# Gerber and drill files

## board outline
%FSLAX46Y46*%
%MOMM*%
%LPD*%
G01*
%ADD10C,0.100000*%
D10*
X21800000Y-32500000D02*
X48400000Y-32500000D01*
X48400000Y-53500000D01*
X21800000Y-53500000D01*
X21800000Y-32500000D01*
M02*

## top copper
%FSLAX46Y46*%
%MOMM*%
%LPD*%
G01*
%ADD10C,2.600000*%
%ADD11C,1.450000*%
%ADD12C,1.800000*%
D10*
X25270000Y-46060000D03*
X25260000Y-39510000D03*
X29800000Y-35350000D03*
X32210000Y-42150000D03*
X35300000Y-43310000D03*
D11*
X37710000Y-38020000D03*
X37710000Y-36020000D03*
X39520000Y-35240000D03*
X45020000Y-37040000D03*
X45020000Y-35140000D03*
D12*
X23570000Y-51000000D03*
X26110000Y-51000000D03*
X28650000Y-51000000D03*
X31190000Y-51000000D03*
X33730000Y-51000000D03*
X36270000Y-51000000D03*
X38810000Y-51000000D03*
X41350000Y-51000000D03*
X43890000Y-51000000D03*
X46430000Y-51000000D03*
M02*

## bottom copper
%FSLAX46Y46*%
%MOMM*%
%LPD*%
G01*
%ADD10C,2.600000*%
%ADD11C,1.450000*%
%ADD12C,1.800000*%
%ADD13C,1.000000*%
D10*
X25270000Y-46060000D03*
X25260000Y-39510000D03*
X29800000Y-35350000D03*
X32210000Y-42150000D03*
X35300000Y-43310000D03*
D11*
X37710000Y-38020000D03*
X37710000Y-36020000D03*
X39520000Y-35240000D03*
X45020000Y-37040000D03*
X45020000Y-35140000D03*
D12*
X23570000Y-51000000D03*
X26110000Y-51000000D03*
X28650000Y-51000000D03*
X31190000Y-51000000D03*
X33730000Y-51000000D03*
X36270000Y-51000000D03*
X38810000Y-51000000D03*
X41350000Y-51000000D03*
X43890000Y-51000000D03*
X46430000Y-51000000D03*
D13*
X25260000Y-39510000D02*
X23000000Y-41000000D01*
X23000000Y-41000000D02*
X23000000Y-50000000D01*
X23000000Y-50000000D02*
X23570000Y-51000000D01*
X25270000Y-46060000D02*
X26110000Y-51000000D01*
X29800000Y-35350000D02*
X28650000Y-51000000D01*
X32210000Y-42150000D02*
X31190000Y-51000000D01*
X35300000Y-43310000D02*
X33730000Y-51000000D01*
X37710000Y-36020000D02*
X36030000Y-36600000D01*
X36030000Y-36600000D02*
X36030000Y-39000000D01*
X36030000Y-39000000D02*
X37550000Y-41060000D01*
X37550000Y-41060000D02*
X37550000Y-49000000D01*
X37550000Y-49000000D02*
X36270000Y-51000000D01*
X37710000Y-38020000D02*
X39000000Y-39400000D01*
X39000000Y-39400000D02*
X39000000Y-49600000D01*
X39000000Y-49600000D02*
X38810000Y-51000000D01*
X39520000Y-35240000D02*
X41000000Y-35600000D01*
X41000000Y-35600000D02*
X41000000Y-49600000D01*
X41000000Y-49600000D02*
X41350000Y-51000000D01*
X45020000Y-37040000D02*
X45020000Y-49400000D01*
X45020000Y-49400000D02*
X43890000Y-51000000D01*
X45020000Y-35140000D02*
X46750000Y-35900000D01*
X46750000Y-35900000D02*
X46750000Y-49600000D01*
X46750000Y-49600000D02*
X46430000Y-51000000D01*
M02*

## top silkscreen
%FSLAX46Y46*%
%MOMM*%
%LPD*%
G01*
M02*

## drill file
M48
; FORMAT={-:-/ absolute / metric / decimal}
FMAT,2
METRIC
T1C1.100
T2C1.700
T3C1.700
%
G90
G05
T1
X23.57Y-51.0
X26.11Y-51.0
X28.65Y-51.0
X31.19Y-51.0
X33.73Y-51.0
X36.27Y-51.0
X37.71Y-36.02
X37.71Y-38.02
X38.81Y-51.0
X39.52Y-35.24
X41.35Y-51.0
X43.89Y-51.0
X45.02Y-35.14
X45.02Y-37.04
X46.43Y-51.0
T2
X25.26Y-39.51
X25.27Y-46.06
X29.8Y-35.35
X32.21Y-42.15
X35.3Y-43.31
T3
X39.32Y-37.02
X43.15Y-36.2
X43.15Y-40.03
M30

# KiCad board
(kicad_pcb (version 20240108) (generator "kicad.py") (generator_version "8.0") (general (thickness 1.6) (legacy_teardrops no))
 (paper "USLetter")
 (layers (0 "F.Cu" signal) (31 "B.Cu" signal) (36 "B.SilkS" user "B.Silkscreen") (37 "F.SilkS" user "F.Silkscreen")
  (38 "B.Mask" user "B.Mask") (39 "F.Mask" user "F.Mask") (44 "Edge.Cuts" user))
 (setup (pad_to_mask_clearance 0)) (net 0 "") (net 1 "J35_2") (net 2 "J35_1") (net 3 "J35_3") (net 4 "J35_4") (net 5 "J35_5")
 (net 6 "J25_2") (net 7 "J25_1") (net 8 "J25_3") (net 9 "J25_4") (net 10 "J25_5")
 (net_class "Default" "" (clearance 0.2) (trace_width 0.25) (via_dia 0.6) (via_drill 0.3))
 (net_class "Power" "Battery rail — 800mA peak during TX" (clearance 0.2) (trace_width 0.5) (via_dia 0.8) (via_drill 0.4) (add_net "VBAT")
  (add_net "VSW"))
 (segment (start 25.26 39.51) (end 23.0 41.0) (width 1.0) (layer "B.Cu") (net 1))
 (segment (start 23.0 41.0) (end 23.0 50.0) (width 1.0) (layer "B.Cu") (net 1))
 (segment (start 23.0 50.0) (end 23.57 51.0) (width 1.0) (layer "B.Cu") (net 1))
 (segment (start 25.27 46.06) (end 26.11 51.0) (width 1.0) (layer "B.Cu") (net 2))
 (segment (start 29.8 35.35) (end 28.65 51.0) (width 1.0) (layer "B.Cu") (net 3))
 (segment (start 32.21 42.15) (end 31.19 51.0) (width 1.0) (layer "B.Cu") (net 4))
 (segment (start 35.3 43.31) (end 33.73 51.0) (width 1.0) (layer "B.Cu") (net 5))
 (segment (start 37.71 36.02) (end 36.03 36.6) (width 1.0) (layer "B.Cu") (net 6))
 (segment (start 36.03 36.6) (end 36.03 39.0) (width 1.0) (layer "B.Cu") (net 6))
 (segment (start 36.03 39.0) (end 37.55 41.06) (width 1.0) (layer "B.Cu") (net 6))
 (segment (start 37.55 41.06) (end 37.55 49.0) (width 1.0) (layer "B.Cu") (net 6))
 (segment (start 37.55 49.0) (end 36.27 51.0) (width 1.0) (layer "B.Cu") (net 6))
 (segment (start 37.71 38.02) (end 39.0 39.4) (width 1.0) (layer "B.Cu") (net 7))
 (segment (start 39.0 39.4) (end 39.0 49.6) (width 1.0) (layer "B.Cu") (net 7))
 (segment (start 39.0 49.6) (end 38.81 51.0) (width 1.0) (layer "B.Cu") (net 7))
 (segment (start 39.52 35.24) (end 41.0 35.6) (width 1.0) (layer "B.Cu") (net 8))
 (segment (start 41.0 35.6) (end 41.0 49.6) (width 1.0) (layer "B.Cu") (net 8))
 (segment (start 41.0 49.6) (end 41.35 51.0) (width 1.0) (layer "B.Cu") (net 8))
 (segment (start 45.02 37.04) (end 45.02 49.4) (width 1.0) (layer "B.Cu") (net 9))
 (segment (start 45.02 49.4) (end 43.89 51.0) (width 1.0) (layer "B.Cu") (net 9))
 (segment (start 45.02 35.14) (end 46.75 35.9) (width 1.0) (layer "B.Cu") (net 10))
 (segment (start 46.75 35.9) (end 46.75 49.6) (width 1.0) (layer "B.Cu") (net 10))
 (segment (start 46.75 49.6) (end 46.43 51.0) (width 1.0) (layer "B.Cu") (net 10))
 (gr_rect (start 21.8 32.5) (end 48.4 53.5) (stroke (width 0.1) (type solid)) (fill none) (layer "Edge.Cuts"))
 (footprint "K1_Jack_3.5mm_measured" (layer "F.Cu") (at 0 0)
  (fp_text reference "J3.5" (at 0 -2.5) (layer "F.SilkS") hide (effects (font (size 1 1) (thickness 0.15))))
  (pad "1" thru_hole circle (at 25.27 46.06) (size 2.6 2.6) (drill 1.7) (layers B.Cu B.Mask) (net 2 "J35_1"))
  (pad "2" thru_hole circle (at 25.26 39.51) (size 2.6 2.6) (drill 1.7) (layers B.Cu B.Mask) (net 1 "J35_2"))
  (pad "3" thru_hole circle (at 29.8 35.35) (size 2.6 2.6) (drill 1.7) (layers B.Cu B.Mask) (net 3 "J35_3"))
  (pad "4" thru_hole circle (at 32.21 42.15) (size 2.6 2.6) (drill 1.7) (layers B.Cu B.Mask) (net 4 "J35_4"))
  (pad "5" thru_hole circle (at 35.3 43.31) (size 2.6 2.6) (drill 1.7) (layers B.Cu B.Mask) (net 5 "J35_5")))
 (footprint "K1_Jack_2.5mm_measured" (layer "F.Cu") (at 0 0)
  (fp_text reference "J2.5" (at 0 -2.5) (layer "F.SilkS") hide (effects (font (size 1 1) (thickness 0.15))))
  (pad "1" thru_hole circle (at 37.71 38.02) (size 1.45 1.45) (drill 1.1) (layers B.Cu B.Mask) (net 7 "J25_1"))
  (pad "2" thru_hole circle (at 37.71 36.02) (size 1.45 1.45) (drill 1.1) (layers B.Cu B.Mask) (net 6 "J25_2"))
  (pad "3" thru_hole circle (at 39.52 35.24) (size 1.45 1.45) (drill 1.1) (layers B.Cu B.Mask) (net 8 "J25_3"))
  (pad "4" thru_hole circle (at 45.02 37.04) (size 1.45 1.45) (drill 1.1) (layers B.Cu B.Mask) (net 9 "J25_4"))
  (pad "5" thru_hole circle (at 45.02 35.14) (size 1.45 1.45) (drill 1.1) (layers B.Cu B.Mask) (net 10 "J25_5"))
  (pad "" np_thru_hole circle (at 43.15 40.03) (size 1.7 1.7) (drill 1.7) (layers *.Cu *.Mask))
  (pad "" np_thru_hole circle (at 43.15 36.2) (size 1.7 1.7) (drill 1.7) (layers *.Cu *.Mask))
  (pad "" np_thru_hole circle (at 39.32 37.02) (size 1.7 1.7) (drill 1.7) (layers *.Cu *.Mask)))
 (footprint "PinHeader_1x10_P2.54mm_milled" (layer "F.Cu") (at 0 0)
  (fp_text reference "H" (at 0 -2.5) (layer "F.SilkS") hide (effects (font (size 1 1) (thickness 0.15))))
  (pad "1" thru_hole circle (at 23.57 51.0) (size 1.8 1.8) (drill 1.1) (layers B.Cu B.Mask) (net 1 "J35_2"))
  (pad "2" thru_hole circle (at 26.11 51.0) (size 1.8 1.8) (drill 1.1) (layers B.Cu B.Mask) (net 2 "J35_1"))
  (pad "3" thru_hole circle (at 28.65 51.0) (size 1.8 1.8) (drill 1.1) (layers B.Cu B.Mask) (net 3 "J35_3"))
  (pad "4" thru_hole circle (at 31.19 51.0) (size 1.8 1.8) (drill 1.1) (layers B.Cu B.Mask) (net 4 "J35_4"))
  (pad "5" thru_hole circle (at 33.73 51.0) (size 1.8 1.8) (drill 1.1) (layers B.Cu B.Mask) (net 5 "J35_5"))
  (pad "6" thru_hole circle (at 36.27 51.0) (size 1.8 1.8) (drill 1.1) (layers B.Cu B.Mask) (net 6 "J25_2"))
  (pad "7" thru_hole circle (at 38.81 51.0) (size 1.8 1.8) (drill 1.1) (layers B.Cu B.Mask) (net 7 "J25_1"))
  (pad "8" thru_hole circle (at 41.35 51.0) (size 1.8 1.8) (drill 1.1) (layers B.Cu B.Mask) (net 8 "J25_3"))
  (pad "9" thru_hole circle (at 43.89 51.0) (size 1.8 1.8) (drill 1.1) (layers B.Cu B.Mask) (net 9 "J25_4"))
  (pad "10" thru_hole circle (at 46.43 51.0) (size 1.8 1.8) (drill 1.1) (layers B.Cu B.Mask) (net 10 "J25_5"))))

